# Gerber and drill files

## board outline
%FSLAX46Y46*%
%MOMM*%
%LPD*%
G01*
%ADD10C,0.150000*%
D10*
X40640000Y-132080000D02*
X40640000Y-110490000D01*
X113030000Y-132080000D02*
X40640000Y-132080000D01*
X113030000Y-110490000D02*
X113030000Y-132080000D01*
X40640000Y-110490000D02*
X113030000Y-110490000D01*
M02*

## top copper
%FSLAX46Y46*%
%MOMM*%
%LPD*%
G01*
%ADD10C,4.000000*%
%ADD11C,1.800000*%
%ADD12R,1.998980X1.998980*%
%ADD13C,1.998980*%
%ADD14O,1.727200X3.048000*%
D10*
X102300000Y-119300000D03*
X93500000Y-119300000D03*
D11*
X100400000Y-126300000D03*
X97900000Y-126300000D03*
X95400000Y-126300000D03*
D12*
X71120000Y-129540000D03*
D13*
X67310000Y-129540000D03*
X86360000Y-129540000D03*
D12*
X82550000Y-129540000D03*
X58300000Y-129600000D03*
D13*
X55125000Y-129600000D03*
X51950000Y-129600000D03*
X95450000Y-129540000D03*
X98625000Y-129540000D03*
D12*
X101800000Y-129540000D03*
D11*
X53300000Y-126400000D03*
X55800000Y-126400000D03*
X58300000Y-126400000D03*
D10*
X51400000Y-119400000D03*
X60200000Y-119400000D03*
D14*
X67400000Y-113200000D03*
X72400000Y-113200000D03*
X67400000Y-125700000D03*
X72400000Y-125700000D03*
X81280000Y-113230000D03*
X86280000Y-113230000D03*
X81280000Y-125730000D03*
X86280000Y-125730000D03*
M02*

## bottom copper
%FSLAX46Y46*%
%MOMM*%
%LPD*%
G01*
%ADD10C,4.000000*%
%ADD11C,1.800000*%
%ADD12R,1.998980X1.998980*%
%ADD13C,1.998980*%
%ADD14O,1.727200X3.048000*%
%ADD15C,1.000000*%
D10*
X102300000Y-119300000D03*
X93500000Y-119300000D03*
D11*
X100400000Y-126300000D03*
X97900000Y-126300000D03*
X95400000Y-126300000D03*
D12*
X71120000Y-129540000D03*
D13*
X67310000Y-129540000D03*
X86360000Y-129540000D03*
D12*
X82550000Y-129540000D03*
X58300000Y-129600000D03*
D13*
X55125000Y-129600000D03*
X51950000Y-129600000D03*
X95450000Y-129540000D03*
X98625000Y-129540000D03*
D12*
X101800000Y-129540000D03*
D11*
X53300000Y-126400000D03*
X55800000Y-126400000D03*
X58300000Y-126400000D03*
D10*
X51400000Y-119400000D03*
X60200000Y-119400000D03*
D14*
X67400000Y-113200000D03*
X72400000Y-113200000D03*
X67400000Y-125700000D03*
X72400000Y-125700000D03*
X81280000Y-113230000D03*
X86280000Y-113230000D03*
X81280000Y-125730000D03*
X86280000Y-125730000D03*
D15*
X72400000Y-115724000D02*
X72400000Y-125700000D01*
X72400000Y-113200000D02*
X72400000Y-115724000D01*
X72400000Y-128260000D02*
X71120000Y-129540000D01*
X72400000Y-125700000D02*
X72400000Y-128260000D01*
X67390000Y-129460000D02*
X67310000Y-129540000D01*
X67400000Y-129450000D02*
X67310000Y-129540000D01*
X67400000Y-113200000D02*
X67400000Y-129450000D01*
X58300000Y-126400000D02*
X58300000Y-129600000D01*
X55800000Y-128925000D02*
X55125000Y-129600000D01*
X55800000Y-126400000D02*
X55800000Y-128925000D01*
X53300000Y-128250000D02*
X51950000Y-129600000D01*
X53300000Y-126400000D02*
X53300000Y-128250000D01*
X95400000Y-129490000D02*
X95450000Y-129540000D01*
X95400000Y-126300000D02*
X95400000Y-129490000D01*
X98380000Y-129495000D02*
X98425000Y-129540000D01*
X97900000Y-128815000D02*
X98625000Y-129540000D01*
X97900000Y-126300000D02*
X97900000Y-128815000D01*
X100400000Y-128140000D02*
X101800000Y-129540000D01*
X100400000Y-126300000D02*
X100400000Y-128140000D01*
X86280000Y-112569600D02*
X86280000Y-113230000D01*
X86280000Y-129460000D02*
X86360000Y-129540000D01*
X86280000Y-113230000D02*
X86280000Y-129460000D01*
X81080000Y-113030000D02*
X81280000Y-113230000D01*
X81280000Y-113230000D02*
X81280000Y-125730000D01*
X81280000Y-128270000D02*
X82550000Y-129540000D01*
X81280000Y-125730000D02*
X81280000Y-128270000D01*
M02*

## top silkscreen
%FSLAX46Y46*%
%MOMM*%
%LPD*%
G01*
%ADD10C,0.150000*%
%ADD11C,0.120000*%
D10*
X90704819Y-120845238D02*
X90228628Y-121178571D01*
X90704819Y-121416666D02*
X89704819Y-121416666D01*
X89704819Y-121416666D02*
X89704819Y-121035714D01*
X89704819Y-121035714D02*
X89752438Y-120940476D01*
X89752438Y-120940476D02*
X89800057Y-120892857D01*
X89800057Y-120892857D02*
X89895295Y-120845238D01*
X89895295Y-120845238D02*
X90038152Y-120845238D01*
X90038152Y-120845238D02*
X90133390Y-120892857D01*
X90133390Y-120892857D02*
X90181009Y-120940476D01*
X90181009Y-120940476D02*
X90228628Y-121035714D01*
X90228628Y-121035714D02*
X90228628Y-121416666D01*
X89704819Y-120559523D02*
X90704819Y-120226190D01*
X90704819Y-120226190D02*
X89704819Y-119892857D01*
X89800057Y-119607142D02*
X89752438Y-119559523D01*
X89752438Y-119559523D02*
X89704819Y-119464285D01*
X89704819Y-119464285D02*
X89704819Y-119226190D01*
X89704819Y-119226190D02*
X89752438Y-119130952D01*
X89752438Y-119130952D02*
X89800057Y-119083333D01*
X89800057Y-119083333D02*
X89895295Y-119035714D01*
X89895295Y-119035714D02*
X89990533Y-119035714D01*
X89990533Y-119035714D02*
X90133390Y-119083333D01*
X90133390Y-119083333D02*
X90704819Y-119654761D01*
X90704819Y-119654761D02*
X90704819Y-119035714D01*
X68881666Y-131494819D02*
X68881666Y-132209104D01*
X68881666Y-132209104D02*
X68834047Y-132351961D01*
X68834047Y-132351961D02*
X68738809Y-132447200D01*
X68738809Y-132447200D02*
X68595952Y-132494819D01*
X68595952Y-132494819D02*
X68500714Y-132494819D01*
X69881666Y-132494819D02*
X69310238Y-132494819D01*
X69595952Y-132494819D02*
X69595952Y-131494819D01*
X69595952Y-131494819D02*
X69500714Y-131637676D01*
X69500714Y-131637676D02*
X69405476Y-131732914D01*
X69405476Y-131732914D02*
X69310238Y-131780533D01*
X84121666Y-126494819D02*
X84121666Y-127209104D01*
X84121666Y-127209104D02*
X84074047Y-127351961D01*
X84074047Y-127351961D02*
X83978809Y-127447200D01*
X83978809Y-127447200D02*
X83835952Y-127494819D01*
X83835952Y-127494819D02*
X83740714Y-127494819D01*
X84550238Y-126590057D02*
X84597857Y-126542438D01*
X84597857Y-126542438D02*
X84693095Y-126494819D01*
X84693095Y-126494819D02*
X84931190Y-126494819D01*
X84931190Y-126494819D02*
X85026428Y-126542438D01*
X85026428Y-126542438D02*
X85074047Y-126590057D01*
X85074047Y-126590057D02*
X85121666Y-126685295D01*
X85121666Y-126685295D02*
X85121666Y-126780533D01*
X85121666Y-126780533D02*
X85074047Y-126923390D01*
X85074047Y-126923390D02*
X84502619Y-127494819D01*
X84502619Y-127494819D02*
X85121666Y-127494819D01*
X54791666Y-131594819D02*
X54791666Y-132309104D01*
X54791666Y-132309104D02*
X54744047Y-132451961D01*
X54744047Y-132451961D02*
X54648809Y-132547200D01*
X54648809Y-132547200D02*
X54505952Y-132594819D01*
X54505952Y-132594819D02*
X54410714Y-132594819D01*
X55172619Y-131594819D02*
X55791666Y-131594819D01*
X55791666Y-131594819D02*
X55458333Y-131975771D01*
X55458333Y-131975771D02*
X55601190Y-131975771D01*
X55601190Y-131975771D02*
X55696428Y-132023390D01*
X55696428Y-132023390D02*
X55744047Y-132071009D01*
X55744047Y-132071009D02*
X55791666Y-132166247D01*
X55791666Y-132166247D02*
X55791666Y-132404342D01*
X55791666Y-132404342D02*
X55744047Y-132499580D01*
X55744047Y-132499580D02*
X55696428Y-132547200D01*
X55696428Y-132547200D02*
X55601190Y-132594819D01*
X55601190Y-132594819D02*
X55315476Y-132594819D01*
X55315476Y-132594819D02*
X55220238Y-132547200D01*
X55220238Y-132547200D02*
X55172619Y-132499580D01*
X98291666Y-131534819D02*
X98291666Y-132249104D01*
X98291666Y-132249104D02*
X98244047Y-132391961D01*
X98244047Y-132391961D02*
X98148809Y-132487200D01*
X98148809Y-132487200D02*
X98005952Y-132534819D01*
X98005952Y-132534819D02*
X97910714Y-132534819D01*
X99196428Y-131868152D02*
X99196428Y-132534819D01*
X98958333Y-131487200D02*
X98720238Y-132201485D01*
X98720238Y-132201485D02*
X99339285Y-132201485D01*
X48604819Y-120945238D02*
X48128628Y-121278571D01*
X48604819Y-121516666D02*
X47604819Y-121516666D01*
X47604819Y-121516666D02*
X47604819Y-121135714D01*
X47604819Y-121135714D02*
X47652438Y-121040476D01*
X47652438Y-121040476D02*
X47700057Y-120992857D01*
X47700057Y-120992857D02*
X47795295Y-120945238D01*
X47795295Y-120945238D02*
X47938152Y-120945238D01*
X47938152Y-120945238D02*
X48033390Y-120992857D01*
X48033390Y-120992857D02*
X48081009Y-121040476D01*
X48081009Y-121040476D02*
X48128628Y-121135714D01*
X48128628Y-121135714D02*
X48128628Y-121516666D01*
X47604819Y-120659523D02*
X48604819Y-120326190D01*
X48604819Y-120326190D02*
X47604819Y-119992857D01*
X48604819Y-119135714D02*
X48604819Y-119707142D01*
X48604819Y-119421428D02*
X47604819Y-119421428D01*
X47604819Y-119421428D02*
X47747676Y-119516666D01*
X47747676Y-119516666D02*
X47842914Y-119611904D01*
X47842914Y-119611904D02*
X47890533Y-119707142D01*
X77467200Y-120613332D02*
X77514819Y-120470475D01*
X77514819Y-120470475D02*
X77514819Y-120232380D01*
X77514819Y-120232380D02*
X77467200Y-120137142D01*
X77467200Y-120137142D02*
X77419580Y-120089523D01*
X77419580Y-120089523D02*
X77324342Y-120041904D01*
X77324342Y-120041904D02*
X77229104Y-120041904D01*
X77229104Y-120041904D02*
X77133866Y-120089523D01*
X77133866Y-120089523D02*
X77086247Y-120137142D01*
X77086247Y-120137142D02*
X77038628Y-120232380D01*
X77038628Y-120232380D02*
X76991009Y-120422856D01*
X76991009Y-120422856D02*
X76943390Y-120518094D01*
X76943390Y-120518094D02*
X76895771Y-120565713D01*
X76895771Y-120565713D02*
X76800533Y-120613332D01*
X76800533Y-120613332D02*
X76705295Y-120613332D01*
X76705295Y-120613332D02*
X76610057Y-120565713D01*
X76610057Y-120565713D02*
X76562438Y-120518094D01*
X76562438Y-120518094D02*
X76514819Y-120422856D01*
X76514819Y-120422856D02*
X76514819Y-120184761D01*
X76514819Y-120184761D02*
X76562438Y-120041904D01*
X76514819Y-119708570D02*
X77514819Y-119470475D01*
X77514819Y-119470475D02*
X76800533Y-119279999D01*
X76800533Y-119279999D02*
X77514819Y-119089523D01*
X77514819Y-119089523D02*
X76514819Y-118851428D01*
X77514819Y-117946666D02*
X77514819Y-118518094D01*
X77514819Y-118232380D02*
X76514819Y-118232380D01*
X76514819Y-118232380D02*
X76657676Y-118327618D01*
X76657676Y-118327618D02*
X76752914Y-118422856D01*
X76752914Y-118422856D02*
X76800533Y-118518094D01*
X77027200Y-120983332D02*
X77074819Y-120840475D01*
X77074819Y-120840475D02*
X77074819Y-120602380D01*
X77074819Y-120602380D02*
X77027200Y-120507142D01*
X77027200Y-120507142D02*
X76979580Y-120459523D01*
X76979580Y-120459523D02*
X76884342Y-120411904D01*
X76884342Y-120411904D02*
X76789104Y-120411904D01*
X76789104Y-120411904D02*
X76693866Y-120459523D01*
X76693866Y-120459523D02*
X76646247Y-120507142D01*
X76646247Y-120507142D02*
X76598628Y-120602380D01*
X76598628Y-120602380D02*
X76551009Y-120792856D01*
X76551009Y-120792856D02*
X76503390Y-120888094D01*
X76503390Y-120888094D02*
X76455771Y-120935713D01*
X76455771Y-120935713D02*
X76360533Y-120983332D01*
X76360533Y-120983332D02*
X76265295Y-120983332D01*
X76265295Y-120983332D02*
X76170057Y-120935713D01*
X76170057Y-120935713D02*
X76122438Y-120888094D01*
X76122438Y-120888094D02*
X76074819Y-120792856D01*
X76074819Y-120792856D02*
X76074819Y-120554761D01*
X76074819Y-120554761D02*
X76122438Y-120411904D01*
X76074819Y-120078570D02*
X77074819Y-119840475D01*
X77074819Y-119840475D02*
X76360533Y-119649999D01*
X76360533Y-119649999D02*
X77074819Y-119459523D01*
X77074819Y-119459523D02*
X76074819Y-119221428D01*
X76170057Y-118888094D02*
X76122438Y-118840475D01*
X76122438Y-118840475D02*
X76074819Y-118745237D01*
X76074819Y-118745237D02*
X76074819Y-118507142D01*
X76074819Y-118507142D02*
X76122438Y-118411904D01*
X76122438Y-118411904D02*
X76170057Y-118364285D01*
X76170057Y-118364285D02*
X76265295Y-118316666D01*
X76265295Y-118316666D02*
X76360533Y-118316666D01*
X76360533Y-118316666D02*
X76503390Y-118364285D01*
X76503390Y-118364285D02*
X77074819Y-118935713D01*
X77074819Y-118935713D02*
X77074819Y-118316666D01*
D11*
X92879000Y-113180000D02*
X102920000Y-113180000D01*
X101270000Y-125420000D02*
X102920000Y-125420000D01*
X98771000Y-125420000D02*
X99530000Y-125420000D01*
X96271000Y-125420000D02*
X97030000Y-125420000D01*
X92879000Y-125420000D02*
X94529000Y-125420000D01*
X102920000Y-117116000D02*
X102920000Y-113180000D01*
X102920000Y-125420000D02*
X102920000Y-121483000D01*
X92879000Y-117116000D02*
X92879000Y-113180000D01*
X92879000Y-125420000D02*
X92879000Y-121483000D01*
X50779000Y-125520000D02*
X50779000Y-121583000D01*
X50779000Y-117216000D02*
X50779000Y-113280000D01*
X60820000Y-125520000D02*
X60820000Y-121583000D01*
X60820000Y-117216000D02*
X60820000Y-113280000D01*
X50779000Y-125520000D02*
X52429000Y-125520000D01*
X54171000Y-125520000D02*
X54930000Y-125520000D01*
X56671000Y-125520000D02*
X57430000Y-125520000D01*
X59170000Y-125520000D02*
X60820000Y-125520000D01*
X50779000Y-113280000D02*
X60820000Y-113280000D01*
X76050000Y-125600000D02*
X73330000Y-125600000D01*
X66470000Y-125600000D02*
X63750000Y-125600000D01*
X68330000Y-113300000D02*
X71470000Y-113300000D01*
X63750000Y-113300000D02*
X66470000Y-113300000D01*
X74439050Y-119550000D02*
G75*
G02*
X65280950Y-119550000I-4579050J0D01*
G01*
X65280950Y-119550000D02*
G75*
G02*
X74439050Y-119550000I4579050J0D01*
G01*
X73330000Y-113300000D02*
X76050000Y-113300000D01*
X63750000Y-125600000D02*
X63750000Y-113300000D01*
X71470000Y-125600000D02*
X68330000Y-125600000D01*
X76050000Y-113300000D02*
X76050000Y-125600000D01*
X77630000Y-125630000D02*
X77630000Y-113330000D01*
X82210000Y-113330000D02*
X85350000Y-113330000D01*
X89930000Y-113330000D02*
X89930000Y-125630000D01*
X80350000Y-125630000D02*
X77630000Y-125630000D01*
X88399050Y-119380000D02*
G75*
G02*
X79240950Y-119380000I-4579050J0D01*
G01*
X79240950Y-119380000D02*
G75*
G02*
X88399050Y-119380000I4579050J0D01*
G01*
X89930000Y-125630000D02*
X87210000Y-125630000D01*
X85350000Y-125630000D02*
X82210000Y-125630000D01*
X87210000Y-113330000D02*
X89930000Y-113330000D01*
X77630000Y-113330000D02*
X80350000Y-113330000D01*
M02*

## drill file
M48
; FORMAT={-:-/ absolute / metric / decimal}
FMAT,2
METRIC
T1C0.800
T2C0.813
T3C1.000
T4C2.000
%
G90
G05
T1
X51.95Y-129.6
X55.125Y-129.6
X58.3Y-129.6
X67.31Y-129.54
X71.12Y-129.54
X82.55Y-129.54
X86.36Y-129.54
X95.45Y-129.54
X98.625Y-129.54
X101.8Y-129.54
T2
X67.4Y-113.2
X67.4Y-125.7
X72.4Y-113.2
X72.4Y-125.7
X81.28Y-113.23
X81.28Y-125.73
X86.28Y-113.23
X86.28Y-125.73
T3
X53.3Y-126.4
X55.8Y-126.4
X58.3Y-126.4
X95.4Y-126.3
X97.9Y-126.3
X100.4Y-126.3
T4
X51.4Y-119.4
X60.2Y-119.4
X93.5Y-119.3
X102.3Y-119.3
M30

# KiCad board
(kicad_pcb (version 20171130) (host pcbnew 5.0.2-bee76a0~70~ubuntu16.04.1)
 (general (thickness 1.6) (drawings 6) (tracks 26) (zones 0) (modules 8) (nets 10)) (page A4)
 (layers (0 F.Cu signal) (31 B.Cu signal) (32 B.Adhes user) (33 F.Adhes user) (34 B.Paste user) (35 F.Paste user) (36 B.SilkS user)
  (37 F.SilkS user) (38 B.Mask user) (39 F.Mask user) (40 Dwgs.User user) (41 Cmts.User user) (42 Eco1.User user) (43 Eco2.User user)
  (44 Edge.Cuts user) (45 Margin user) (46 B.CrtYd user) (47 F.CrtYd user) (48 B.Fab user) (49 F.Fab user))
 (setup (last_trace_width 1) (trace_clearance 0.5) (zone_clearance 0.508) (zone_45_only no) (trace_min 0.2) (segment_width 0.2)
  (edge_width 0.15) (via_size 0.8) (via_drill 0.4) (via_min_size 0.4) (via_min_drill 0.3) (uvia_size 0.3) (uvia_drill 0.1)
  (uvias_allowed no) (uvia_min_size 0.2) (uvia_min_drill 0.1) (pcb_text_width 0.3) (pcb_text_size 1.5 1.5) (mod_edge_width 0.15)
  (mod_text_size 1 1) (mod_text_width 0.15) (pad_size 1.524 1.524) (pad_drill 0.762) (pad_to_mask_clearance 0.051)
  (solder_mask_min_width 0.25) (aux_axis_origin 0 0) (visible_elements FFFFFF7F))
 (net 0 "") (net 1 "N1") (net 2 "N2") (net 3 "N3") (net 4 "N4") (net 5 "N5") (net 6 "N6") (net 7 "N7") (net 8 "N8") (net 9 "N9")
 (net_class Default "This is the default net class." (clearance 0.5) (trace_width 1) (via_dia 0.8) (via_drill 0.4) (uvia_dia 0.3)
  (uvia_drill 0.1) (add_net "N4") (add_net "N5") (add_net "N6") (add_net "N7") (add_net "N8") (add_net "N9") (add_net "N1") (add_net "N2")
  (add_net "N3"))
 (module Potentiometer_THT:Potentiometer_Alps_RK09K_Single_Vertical (layer F.Cu) (at 100.4 126.3 90)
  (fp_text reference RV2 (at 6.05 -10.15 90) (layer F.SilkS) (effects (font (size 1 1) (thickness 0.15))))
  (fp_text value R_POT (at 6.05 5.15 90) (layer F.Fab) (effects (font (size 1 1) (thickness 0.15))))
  (fp_line (start 13.12 -7.521) (end 13.12 2.52) (layer F.SilkS) (width 0.12))
  (fp_line (start 0.88 0.87) (end 0.88 2.52) (layer F.SilkS) (width 0.12))
  (fp_line (start 0.88 -1.629) (end 0.88 -0.87) (layer F.SilkS) (width 0.12))
  (fp_line (start 0.88 -4.129) (end 0.88 -3.37) (layer F.SilkS) (width 0.12))
  (fp_line (start 0.88 -7.521) (end 0.88 -5.871) (layer F.SilkS) (width 0.12))
  (fp_line (start 9.184 2.52) (end 13.12 2.52) (layer F.SilkS) (width 0.12))
  (fp_line (start 0.88 2.52) (end 4.817 2.52) (layer F.SilkS) (width 0.12))
  (fp_line (start 9.184 -7.521) (end 13.12 -7.521) (layer F.SilkS) (width 0.12))
  (fp_line (start 0.88 -7.521) (end 4.817 -7.521) (layer F.SilkS) (width 0.12))
  (pad "" np_thru_hole circle (at 7 1.9 90) (size 4 4) (drill 2) (layers *.Cu *.Mask))
  (pad "" np_thru_hole circle (at 7 -6.9 90) (size 4 4) (drill 2) (layers *.Cu *.Mask))
  (pad 1 thru_hole circle (at 0 0 90) (size 1.8 1.8) (drill 1) (layers *.Cu *.Mask) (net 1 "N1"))
  (pad 2 thru_hole circle (at 0 -2.5 90) (size 1.8 1.8) (drill 1) (layers *.Cu *.Mask) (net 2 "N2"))
  (pad 3 thru_hole circle (at 0 -5 90) (size 1.8 1.8) (drill 1) (layers *.Cu *.Mask) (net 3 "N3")))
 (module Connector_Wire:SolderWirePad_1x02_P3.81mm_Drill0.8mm (layer F.Cu) (at 71.12 129.54 180)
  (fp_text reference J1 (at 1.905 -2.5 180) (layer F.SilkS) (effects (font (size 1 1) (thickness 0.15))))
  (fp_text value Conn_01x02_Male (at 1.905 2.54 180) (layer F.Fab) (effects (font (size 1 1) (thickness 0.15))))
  (pad 1 thru_hole rect (at 0 0 180) (size 1.99898 1.99898) (drill 0.8001) (layers *.Cu *.Mask) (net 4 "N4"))
  (pad 2 thru_hole circle (at 3.81 0 180) (size 1.99898 1.99898) (drill 0.8001) (layers *.Cu *.Mask) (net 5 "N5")))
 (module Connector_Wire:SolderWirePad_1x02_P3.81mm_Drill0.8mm (layer F.Cu) (at 82.55 129.54)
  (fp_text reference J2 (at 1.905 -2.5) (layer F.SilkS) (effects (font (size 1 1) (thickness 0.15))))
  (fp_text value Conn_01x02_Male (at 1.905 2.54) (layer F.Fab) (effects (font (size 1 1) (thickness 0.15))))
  (pad 2 thru_hole circle (at 3.81 0) (size 1.99898 1.99898) (drill 0.8001) (layers *.Cu *.Mask) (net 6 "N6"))
  (pad 1 thru_hole rect (at 0 0) (size 1.99898 1.99898) (drill 0.8001) (layers *.Cu *.Mask) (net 4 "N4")))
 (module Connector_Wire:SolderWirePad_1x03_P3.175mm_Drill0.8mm (layer F.Cu) (at 58.3 129.6 180)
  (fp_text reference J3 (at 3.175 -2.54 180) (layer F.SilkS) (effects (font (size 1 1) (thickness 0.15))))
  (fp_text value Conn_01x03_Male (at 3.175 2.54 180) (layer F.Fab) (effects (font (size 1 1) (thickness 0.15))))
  (pad 1 thru_hole rect (at 0 0 180) (size 1.99898 1.99898) (drill 0.8001) (layers *.Cu *.Mask) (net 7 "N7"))
  (pad 2 thru_hole circle (at 3.175 0 180) (size 1.99898 1.99898) (drill 0.8001) (layers *.Cu *.Mask) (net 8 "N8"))
  (pad 3 thru_hole circle (at 6.35 0 180) (size 1.99898 1.99898) (drill 0.8001) (layers *.Cu *.Mask) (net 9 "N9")))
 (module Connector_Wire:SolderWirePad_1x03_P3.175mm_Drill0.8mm (layer F.Cu) (at 101.8 129.54 180)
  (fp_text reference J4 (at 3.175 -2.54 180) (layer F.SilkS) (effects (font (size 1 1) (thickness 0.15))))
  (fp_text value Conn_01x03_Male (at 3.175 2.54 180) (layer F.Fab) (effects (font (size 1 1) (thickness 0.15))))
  (pad 3 thru_hole circle (at 6.35 0 180) (size 1.99898 1.99898) (drill 0.8001) (layers *.Cu *.Mask) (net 3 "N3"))
  (pad 2 thru_hole circle (at 3.175 0 180) (size 1.99898 1.99898) (drill 0.8001) (layers *.Cu *.Mask) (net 2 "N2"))
  (pad 1 thru_hole rect (at 0 0 180) (size 1.99898 1.99898) (drill 0.8001) (layers *.Cu *.Mask) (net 1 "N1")))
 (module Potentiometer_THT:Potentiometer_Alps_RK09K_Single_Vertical (layer F.Cu) (at 58.3 126.4 90)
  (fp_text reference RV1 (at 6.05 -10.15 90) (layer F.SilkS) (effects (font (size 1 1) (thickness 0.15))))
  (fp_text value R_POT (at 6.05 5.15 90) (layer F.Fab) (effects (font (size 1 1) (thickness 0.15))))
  (fp_line (start 0.88 -7.521) (end 4.817 -7.521) (layer F.SilkS) (width 0.12))
  (fp_line (start 9.184 -7.521) (end 13.12 -7.521) (layer F.SilkS) (width 0.12))
  (fp_line (start 0.88 2.52) (end 4.817 2.52) (layer F.SilkS) (width 0.12))
  (fp_line (start 9.184 2.52) (end 13.12 2.52) (layer F.SilkS) (width 0.12))
  (fp_line (start 0.88 -7.521) (end 0.88 -5.871) (layer F.SilkS) (width 0.12))
  (fp_line (start 0.88 -4.129) (end 0.88 -3.37) (layer F.SilkS) (width 0.12))
  (fp_line (start 0.88 -1.629) (end 0.88 -0.87) (layer F.SilkS) (width 0.12))
  (fp_line (start 0.88 0.87) (end 0.88 2.52) (layer F.SilkS) (width 0.12))
  (fp_line (start 13.12 -7.521) (end 13.12 2.52) (layer F.SilkS) (width 0.12))
  (pad 3 thru_hole circle (at 0 -5 90) (size 1.8 1.8) (drill 1) (layers *.Cu *.Mask) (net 9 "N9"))
  (pad 2 thru_hole circle (at 0 -2.5 90) (size 1.8 1.8) (drill 1) (layers *.Cu *.Mask) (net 8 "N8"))
  (pad 1 thru_hole circle (at 0 0 90) (size 1.8 1.8) (drill 1) (layers *.Cu *.Mask) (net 7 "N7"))
  (pad "" np_thru_hole circle (at 7 -6.9 90) (size 4 4) (drill 2) (layers *.Cu *.Mask))
  (pad "" np_thru_hole circle (at 7 1.9 90) (size 4 4) (drill 2) (layers *.Cu *.Mask)))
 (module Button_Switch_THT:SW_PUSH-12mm (layer F.Cu) (at 72.4 113.2 270)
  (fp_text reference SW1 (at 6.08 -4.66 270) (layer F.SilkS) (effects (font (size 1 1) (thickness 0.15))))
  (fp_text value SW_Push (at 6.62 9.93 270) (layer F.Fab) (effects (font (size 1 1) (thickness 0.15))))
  (fp_line (start 12.4 -3.65) (end 12.4 -0.93) (layer F.SilkS) (width 0.12))
  (fp_line (start 12.4 5.93) (end 12.4 8.65) (layer F.SilkS) (width 0.12))
  (fp_line (start 0.1 4.07) (end 0.1 0.93) (layer F.SilkS) (width 0.12))
  (fp_line (start 0.1 8.65) (end 0.1 5.93) (layer F.SilkS) (width 0.12))
  (fp_circle (center 6.35 2.54) (end 10.16 5.08) (layer F.SilkS) (width 0.12))
  (fp_line (start 0.1 -0.93) (end 0.1 -3.65) (layer F.SilkS) (width 0.12))
  (fp_line (start 12.4 8.65) (end 0.1 8.65) (layer F.SilkS) (width 0.12))
  (fp_line (start 12.4 0.93) (end 12.4 4.07) (layer F.SilkS) (width 0.12))
  (fp_line (start 0.1 -3.65) (end 12.4 -3.65) (layer F.SilkS) (width 0.12))
  (pad 2 thru_hole oval (at 0 5 270) (size 3.048 1.7272) (drill 0.8128) (layers *.Cu *.Mask) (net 5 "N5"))
  (pad 1 thru_hole oval (at 0 0 270) (size 3.048 1.7272) (drill 0.8128) (layers *.Cu *.Mask) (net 4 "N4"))
  (pad 2 thru_hole oval (at 12.5 5 270) (size 3.048 1.7272) (drill 0.8128) (layers *.Cu *.Mask) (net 5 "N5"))
  (pad 1 thru_hole oval (at 12.5 0 270) (size 3.048 1.7272) (drill 0.8128) (layers *.Cu *.Mask) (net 4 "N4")))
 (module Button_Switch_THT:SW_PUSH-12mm (layer F.Cu) (at 81.28 125.73 90)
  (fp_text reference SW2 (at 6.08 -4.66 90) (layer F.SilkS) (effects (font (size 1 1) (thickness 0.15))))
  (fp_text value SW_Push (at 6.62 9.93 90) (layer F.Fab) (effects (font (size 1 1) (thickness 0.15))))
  (fp_line (start 0.1 -3.65) (end 12.4 -3.65) (layer F.SilkS) (width 0.12))
  (fp_line (start 12.4 0.93) (end 12.4 4.07) (layer F.SilkS) (width 0.12))
  (fp_line (start 12.4 8.65) (end 0.1 8.65) (layer F.SilkS) (width 0.12))
  (fp_line (start 0.1 -0.93) (end 0.1 -3.65) (layer F.SilkS) (width 0.12))
  (fp_circle (center 6.35 2.54) (end 10.16 5.08) (layer F.SilkS) (width 0.12))
  (fp_line (start 0.1 8.65) (end 0.1 5.93) (layer F.SilkS) (width 0.12))
  (fp_line (start 0.1 4.07) (end 0.1 0.93) (layer F.SilkS) (width 0.12))
  (fp_line (start 12.4 5.93) (end 12.4 8.65) (layer F.SilkS) (width 0.12))
  (fp_line (start 12.4 -3.65) (end 12.4 -0.93) (layer F.SilkS) (width 0.12))
  (pad 1 thru_hole oval (at 12.5 0 90) (size 3.048 1.7272) (drill 0.8128) (layers *.Cu *.Mask) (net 4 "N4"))
  (pad 2 thru_hole oval (at 12.5 5 90) (size 3.048 1.7272) (drill 0.8128) (layers *.Cu *.Mask) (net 6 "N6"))
  (pad 1 thru_hole oval (at 0 0 90) (size 3.048 1.7272) (drill 0.8128) (layers *.Cu *.Mask) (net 4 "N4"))
  (pad 2 thru_hole oval (at 0 5 90) (size 3.048 1.7272) (drill 0.8128) (layers *.Cu *.Mask) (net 6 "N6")))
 (gr_line (start 40.64 132.08) (end 40.64 110.49) (layer Edge.Cuts) (width 0.15))
 (gr_line (start 113.03 132.08) (end 40.64 132.08) (layer Edge.Cuts) (width 0.15))
 (gr_line (start 113.03 110.49) (end 113.03 132.08) (layer Edge.Cuts) (width 0.15))
 (gr_line (start 40.64 110.49) (end 113.03 110.49) (layer Edge.Cuts) (width 0.15))
 (segment (start 72.4 115.724) (end 72.4 125.7) (width 1) (layer B.Cu) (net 4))
 (segment (start 72.4 113.2) (end 72.4 115.724) (width 1) (layer B.Cu) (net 4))
 (segment (start 72.4 128.26) (end 71.12 129.54) (width 1) (layer B.Cu) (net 4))
 (segment (start 72.4 125.7) (end 72.4 128.26) (width 1) (layer B.Cu) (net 4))
 (segment (start 67.39 129.46) (end 67.31 129.54) (width 1) (layer B.Cu) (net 5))
 (segment (start 67.4 129.45) (end 67.31 129.54) (width 1) (layer B.Cu) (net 5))
 (segment (start 67.4 113.2) (end 67.4 129.45) (width 1) (layer B.Cu) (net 5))
 (segment (start 58.3 126.4) (end 58.3 129.6) (width 1) (layer B.Cu) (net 7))
 (segment (start 55.8 128.925) (end 55.125 129.6) (width 1) (layer B.Cu) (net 8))
 (segment (start 55.8 126.4) (end 55.8 128.925) (width 1) (layer B.Cu) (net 8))
 (segment (start 53.3 128.25) (end 51.95 129.6) (width 1) (layer B.Cu) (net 9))
 (segment (start 53.3 126.4) (end 53.3 128.25) (width 1) (layer B.Cu) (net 9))
 (segment (start 95.4 129.49) (end 95.45 129.54) (width 1) (layer B.Cu) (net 3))
 (segment (start 95.4 126.3) (end 95.4 129.49) (width 1) (layer B.Cu) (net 3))
 (segment (start 98.38 129.495) (end 98.425 129.54) (width 1) (layer B.Cu) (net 2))
 (segment (start 97.9 128.815) (end 98.625 129.54) (width 1) (layer B.Cu) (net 2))
 (segment (start 97.9 126.3) (end 97.9 128.815) (width 1) (layer B.Cu) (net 2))
 (segment (start 100.4 128.14) (end 101.8 129.54) (width 1) (layer B.Cu) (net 1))
 (segment (start 100.4 126.3) (end 100.4 128.14) (width 1) (layer B.Cu) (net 1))
 (segment (start 86.28 112.5696) (end 86.28 113.23) (width 1) (layer B.Cu) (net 6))
 (segment (start 86.28 129.46) (end 86.36 129.54) (width 1) (layer B.Cu) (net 6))
 (segment (start 86.28 113.23) (end 86.28 129.46) (width 1) (layer B.Cu) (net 6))
 (segment (start 81.08 113.03) (end 81.28 113.23) (width 1) (layer B.Cu) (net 4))
 (segment (start 81.28 113.23) (end 81.28 125.73) (width 1) (layer B.Cu) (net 4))
 (segment (start 81.28 128.27) (end 82.55 129.54) (width 1) (layer B.Cu) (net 4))
 (segment (start 81.28 125.73) (end 81.28 128.27) (width 1) (layer B.Cu) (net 4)))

